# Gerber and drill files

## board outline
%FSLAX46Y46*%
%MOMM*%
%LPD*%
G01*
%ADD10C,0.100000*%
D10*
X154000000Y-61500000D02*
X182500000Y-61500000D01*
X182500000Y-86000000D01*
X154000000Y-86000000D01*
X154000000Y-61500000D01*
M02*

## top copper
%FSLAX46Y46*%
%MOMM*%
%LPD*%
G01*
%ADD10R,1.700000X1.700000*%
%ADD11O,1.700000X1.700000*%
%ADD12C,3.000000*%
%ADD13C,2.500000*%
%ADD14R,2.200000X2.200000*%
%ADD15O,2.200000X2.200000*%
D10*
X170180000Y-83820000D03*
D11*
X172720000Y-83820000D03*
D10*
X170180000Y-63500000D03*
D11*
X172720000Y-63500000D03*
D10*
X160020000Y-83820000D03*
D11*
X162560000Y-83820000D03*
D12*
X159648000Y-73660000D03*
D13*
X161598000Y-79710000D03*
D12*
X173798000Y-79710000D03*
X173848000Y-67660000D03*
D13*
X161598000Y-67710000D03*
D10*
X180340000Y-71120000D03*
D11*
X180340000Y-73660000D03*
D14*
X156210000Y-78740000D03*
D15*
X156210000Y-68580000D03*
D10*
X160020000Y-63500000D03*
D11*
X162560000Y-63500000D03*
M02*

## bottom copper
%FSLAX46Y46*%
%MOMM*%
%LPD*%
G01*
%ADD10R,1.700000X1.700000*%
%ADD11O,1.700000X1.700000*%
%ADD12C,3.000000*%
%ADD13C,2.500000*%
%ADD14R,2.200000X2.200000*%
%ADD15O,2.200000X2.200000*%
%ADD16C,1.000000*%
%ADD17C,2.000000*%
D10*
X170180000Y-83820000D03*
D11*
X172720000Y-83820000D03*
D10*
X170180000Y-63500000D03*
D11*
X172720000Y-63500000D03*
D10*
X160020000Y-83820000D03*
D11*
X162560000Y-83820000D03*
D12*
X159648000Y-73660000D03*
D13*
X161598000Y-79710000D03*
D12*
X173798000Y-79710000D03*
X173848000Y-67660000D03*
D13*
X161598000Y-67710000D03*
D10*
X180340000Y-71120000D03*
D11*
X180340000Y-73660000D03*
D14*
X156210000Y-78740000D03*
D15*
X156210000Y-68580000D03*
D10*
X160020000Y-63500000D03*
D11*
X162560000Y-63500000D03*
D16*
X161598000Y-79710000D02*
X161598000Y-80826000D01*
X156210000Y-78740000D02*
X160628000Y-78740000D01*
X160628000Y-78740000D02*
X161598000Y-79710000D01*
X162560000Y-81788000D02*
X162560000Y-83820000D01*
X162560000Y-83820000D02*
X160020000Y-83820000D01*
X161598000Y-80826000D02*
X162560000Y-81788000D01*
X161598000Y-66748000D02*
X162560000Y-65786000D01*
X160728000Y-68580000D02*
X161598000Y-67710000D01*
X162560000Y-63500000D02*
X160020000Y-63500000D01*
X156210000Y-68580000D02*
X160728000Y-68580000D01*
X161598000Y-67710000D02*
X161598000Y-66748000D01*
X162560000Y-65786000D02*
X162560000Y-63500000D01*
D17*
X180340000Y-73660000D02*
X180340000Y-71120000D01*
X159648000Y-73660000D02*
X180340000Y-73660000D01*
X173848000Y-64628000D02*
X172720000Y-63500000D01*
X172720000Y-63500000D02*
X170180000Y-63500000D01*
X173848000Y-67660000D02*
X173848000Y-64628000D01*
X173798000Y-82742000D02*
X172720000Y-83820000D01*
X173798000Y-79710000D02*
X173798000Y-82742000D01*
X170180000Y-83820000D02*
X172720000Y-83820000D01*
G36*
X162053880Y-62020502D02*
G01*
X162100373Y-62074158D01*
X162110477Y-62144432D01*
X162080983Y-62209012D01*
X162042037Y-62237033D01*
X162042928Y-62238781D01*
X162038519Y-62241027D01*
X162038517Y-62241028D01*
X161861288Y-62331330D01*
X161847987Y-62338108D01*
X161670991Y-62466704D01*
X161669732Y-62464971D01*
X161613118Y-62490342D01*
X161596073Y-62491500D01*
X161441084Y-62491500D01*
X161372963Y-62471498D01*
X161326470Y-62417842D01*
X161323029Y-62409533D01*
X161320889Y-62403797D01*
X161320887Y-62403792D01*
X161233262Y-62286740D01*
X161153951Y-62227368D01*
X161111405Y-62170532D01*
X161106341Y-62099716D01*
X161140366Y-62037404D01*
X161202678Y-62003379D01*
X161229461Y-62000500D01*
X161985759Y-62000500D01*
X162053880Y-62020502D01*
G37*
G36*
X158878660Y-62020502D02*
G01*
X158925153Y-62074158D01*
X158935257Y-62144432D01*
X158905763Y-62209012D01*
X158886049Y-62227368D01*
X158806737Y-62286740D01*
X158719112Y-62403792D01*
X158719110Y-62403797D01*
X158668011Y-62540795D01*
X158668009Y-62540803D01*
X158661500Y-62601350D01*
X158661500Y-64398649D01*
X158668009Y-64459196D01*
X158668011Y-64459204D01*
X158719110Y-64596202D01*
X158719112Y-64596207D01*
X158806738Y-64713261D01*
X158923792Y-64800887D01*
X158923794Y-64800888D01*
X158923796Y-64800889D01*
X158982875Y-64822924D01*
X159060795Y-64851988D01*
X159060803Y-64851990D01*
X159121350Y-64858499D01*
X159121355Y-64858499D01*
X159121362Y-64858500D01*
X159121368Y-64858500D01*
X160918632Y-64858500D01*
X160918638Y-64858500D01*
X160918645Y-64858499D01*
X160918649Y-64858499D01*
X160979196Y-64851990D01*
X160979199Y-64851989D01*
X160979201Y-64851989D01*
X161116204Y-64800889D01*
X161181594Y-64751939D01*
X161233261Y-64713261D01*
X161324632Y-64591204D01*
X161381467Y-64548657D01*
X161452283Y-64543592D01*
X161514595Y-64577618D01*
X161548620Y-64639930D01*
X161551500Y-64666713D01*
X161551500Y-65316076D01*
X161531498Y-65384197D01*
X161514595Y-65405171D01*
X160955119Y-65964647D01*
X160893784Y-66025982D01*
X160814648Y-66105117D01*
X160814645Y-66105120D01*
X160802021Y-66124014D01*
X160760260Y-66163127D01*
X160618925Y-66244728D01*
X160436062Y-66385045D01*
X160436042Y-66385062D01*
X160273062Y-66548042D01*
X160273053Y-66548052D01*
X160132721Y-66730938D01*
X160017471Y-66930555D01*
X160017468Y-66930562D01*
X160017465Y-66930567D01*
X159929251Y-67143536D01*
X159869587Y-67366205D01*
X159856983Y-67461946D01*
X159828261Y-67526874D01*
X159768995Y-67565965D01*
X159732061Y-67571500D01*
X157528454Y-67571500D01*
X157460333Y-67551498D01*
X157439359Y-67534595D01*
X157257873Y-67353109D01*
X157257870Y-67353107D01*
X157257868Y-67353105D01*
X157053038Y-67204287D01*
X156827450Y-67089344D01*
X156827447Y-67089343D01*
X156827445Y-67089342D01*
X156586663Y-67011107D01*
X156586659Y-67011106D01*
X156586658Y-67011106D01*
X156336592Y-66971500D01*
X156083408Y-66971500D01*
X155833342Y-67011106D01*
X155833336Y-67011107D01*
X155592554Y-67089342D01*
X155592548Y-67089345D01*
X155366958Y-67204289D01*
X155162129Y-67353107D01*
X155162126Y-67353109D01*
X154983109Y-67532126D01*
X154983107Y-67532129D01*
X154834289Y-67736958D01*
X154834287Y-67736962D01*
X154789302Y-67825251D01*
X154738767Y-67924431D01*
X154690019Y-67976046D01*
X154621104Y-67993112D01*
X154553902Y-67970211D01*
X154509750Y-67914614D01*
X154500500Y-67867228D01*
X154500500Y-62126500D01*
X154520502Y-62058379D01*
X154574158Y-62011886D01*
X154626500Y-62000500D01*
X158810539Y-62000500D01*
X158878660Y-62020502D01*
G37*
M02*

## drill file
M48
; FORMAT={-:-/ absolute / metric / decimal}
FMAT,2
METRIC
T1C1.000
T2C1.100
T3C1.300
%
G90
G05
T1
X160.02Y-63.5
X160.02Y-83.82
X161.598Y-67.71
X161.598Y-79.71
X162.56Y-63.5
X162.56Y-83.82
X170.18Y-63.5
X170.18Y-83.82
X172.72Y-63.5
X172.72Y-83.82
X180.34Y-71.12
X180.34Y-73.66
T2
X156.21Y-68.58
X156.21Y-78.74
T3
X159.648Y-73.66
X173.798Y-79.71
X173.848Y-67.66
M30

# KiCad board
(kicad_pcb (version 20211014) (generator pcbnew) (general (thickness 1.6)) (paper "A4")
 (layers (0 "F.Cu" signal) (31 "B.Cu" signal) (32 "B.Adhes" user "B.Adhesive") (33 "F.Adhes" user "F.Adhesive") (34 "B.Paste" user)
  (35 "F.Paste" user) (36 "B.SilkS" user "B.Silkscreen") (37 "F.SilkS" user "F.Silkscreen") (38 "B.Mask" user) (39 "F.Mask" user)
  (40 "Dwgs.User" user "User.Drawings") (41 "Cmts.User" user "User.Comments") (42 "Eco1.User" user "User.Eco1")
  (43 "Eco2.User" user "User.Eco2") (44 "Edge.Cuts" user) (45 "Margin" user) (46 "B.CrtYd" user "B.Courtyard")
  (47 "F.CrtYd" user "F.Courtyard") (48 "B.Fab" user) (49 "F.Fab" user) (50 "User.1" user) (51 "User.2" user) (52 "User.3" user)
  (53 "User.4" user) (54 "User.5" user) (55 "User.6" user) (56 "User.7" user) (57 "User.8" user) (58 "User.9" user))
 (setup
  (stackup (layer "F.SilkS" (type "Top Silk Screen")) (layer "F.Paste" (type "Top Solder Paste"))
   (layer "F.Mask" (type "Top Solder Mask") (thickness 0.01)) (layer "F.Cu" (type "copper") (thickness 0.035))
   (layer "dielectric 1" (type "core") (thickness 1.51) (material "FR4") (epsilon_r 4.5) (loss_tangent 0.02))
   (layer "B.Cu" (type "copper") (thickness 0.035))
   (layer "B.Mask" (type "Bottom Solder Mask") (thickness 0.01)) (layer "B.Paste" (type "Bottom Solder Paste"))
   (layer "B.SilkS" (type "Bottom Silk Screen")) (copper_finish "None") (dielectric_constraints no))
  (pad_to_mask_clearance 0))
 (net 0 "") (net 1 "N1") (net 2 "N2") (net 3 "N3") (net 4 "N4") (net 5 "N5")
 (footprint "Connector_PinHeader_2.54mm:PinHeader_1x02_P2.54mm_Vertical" (layer "F.Cu") (at 170.18 83.82 90)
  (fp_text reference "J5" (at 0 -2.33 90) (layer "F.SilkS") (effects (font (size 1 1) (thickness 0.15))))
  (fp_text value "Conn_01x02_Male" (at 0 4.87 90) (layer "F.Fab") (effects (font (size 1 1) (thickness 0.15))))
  (pad "1" thru_hole rect (at 0 0 90) (size 1.7 1.7) (drill 1) (layers *.Cu *.Mask) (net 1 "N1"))
  (pad "2" thru_hole oval (at 0 2.54 90) (size 1.7 1.7) (drill 1) (layers *.Cu *.Mask) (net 1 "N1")))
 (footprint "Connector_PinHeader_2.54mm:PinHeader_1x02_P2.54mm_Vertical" (layer "F.Cu") (at 170.18 63.5 90)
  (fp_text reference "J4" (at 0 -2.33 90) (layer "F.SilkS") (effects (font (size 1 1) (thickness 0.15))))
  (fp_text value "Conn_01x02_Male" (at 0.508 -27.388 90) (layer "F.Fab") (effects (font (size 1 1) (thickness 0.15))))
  (pad "1" thru_hole rect (at 0 0 90) (size 1.7 1.7) (drill 1) (layers *.Cu *.Mask) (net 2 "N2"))
  (pad "2" thru_hole oval (at 0 2.54 90) (size 1.7 1.7) (drill 1) (layers *.Cu *.Mask) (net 2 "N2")))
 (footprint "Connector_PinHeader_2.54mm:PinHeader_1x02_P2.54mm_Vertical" (layer "F.Cu") (at 160.02 83.82 90)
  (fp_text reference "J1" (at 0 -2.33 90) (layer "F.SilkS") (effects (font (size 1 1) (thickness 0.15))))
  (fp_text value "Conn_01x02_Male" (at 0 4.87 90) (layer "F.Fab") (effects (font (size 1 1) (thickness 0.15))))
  (pad "1" thru_hole rect (at 0 0 90) (size 1.7 1.7) (drill 1) (layers *.Cu *.Mask) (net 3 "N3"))
  (pad "2" thru_hole oval (at 0 2.54 90) (size 1.7 1.7) (drill 1) (layers *.Cu *.Mask) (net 3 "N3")))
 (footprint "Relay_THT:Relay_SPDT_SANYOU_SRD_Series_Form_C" (layer "F.Cu") (at 159.648 73.66)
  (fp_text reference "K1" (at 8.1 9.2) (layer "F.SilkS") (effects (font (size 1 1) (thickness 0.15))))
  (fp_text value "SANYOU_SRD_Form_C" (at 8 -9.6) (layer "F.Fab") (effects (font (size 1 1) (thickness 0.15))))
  (pad "1" thru_hole circle (at 0 0 90) (size 3 3) (drill 1.3) (layers *.Cu *.Mask) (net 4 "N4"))
  (pad "2" thru_hole circle (at 1.95 6.05 90) (size 2.5 2.5) (drill 1) (layers *.Cu *.Mask) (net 3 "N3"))
  (pad "3" thru_hole circle (at 14.15 6.05 90) (size 3 3) (drill 1.3) (layers *.Cu *.Mask) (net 1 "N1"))
  (pad "4" thru_hole circle (at 14.2 -6 90) (size 3 3) (drill 1.3) (layers *.Cu *.Mask) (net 2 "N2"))
  (pad "5" thru_hole circle (at 1.95 -5.95 90) (size 2.5 2.5) (drill 1) (layers *.Cu *.Mask) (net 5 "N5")))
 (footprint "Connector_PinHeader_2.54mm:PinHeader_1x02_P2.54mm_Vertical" (layer "F.Cu") (at 180.34 71.12)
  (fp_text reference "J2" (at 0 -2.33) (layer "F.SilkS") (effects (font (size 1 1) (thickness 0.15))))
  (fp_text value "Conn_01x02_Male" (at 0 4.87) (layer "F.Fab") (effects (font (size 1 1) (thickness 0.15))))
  (pad "1" thru_hole rect (at 0 0) (size 1.7 1.7) (drill 1) (layers *.Cu *.Mask) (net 4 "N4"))
  (pad "2" thru_hole oval (at 0 2.54) (size 1.7 1.7) (drill 1) (layers *.Cu *.Mask) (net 4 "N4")))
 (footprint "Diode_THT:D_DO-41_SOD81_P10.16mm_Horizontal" (layer "F.Cu") (at 156.21 78.74 90)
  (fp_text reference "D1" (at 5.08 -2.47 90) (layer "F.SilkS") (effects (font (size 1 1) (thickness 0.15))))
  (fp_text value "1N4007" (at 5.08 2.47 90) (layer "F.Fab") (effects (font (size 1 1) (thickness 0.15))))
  (pad "1" thru_hole rect (at 0 0 90) (size 2.2 2.2) (drill 1.1) (layers *.Cu *.Mask) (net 3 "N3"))
  (pad "2" thru_hole oval (at 10.16 0 90) (size 2.2 2.2) (drill 1.1) (layers *.Cu *.Mask) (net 5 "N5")))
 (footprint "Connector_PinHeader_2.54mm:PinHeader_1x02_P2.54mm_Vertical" (layer "F.Cu") (at 160.02 63.5 90)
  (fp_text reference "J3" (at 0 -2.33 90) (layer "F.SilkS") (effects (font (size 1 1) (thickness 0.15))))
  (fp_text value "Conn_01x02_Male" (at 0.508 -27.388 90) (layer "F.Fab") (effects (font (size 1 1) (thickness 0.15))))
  (pad "1" thru_hole rect (at 0 0 90) (size 1.7 1.7) (drill 1) (layers *.Cu *.Mask) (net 5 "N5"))
  (pad "2" thru_hole oval (at 0 2.54 90) (size 1.7 1.7) (drill 1) (layers *.Cu *.Mask) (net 5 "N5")))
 (gr_rect (start 154 61.5) (end 182.5 86) (layer "Edge.Cuts") (width 0.1) (fill none))
 (segment (start 161.598 79.71) (end 161.598 80.826) (width 1) (layer "B.Cu") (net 3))
 (segment (start 156.21 78.74) (end 160.628 78.74) (width 1) (layer "B.Cu") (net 3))
 (segment (start 160.628 78.74) (end 161.598 79.71) (width 1) (layer "B.Cu") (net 3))
 (segment (start 162.56 81.788) (end 162.56 83.82) (width 1) (layer "B.Cu") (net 3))
 (segment (start 162.56 83.82) (end 160.02 83.82) (width 1) (layer "B.Cu") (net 3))
 (segment (start 161.598 80.826) (end 162.56 81.788) (width 1) (layer "B.Cu") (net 3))
 (segment (start 161.598 66.748) (end 162.56 65.786) (width 1) (layer "B.Cu") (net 5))
 (segment (start 160.728 68.58) (end 161.598 67.71) (width 1) (layer "B.Cu") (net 5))
 (segment (start 162.56 63.5) (end 160.02 63.5) (width 1) (layer "B.Cu") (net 5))
 (segment (start 156.21 68.58) (end 160.728 68.58) (width 1) (layer "B.Cu") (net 5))
 (segment (start 161.598 67.71) (end 161.598 66.748) (width 1) (layer "B.Cu") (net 5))
 (segment (start 162.56 65.786) (end 162.56 63.5) (width 1) (layer "B.Cu") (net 5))
 (segment (start 180.34 73.66) (end 180.34 71.12) (width 2) (layer "B.Cu") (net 4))
 (segment (start 159.648 73.66) (end 180.34 73.66) (width 2) (layer "B.Cu") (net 4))
 (segment (start 173.848 64.628) (end 172.72 63.5) (width 2) (layer "B.Cu") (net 2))
 (segment (start 172.72 63.5) (end 170.18 63.5) (width 2) (layer "B.Cu") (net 2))
 (segment (start 173.848 67.66) (end 173.848 64.628) (width 2) (layer "B.Cu") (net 2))
 (segment (start 173.798 82.742) (end 172.72 83.82) (width 2) (layer "B.Cu") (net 1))
 (segment (start 173.798 79.71) (end 173.798 82.742) (width 2) (layer "B.Cu") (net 1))
 (segment (start 170.18 83.82) (end 172.72 83.82) (width 2) (layer "B.Cu") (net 1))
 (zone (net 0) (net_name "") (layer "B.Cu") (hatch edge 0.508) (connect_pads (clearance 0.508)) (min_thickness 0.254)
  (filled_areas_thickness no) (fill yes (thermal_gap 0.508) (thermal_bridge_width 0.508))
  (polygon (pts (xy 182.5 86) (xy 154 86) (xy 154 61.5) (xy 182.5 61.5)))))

